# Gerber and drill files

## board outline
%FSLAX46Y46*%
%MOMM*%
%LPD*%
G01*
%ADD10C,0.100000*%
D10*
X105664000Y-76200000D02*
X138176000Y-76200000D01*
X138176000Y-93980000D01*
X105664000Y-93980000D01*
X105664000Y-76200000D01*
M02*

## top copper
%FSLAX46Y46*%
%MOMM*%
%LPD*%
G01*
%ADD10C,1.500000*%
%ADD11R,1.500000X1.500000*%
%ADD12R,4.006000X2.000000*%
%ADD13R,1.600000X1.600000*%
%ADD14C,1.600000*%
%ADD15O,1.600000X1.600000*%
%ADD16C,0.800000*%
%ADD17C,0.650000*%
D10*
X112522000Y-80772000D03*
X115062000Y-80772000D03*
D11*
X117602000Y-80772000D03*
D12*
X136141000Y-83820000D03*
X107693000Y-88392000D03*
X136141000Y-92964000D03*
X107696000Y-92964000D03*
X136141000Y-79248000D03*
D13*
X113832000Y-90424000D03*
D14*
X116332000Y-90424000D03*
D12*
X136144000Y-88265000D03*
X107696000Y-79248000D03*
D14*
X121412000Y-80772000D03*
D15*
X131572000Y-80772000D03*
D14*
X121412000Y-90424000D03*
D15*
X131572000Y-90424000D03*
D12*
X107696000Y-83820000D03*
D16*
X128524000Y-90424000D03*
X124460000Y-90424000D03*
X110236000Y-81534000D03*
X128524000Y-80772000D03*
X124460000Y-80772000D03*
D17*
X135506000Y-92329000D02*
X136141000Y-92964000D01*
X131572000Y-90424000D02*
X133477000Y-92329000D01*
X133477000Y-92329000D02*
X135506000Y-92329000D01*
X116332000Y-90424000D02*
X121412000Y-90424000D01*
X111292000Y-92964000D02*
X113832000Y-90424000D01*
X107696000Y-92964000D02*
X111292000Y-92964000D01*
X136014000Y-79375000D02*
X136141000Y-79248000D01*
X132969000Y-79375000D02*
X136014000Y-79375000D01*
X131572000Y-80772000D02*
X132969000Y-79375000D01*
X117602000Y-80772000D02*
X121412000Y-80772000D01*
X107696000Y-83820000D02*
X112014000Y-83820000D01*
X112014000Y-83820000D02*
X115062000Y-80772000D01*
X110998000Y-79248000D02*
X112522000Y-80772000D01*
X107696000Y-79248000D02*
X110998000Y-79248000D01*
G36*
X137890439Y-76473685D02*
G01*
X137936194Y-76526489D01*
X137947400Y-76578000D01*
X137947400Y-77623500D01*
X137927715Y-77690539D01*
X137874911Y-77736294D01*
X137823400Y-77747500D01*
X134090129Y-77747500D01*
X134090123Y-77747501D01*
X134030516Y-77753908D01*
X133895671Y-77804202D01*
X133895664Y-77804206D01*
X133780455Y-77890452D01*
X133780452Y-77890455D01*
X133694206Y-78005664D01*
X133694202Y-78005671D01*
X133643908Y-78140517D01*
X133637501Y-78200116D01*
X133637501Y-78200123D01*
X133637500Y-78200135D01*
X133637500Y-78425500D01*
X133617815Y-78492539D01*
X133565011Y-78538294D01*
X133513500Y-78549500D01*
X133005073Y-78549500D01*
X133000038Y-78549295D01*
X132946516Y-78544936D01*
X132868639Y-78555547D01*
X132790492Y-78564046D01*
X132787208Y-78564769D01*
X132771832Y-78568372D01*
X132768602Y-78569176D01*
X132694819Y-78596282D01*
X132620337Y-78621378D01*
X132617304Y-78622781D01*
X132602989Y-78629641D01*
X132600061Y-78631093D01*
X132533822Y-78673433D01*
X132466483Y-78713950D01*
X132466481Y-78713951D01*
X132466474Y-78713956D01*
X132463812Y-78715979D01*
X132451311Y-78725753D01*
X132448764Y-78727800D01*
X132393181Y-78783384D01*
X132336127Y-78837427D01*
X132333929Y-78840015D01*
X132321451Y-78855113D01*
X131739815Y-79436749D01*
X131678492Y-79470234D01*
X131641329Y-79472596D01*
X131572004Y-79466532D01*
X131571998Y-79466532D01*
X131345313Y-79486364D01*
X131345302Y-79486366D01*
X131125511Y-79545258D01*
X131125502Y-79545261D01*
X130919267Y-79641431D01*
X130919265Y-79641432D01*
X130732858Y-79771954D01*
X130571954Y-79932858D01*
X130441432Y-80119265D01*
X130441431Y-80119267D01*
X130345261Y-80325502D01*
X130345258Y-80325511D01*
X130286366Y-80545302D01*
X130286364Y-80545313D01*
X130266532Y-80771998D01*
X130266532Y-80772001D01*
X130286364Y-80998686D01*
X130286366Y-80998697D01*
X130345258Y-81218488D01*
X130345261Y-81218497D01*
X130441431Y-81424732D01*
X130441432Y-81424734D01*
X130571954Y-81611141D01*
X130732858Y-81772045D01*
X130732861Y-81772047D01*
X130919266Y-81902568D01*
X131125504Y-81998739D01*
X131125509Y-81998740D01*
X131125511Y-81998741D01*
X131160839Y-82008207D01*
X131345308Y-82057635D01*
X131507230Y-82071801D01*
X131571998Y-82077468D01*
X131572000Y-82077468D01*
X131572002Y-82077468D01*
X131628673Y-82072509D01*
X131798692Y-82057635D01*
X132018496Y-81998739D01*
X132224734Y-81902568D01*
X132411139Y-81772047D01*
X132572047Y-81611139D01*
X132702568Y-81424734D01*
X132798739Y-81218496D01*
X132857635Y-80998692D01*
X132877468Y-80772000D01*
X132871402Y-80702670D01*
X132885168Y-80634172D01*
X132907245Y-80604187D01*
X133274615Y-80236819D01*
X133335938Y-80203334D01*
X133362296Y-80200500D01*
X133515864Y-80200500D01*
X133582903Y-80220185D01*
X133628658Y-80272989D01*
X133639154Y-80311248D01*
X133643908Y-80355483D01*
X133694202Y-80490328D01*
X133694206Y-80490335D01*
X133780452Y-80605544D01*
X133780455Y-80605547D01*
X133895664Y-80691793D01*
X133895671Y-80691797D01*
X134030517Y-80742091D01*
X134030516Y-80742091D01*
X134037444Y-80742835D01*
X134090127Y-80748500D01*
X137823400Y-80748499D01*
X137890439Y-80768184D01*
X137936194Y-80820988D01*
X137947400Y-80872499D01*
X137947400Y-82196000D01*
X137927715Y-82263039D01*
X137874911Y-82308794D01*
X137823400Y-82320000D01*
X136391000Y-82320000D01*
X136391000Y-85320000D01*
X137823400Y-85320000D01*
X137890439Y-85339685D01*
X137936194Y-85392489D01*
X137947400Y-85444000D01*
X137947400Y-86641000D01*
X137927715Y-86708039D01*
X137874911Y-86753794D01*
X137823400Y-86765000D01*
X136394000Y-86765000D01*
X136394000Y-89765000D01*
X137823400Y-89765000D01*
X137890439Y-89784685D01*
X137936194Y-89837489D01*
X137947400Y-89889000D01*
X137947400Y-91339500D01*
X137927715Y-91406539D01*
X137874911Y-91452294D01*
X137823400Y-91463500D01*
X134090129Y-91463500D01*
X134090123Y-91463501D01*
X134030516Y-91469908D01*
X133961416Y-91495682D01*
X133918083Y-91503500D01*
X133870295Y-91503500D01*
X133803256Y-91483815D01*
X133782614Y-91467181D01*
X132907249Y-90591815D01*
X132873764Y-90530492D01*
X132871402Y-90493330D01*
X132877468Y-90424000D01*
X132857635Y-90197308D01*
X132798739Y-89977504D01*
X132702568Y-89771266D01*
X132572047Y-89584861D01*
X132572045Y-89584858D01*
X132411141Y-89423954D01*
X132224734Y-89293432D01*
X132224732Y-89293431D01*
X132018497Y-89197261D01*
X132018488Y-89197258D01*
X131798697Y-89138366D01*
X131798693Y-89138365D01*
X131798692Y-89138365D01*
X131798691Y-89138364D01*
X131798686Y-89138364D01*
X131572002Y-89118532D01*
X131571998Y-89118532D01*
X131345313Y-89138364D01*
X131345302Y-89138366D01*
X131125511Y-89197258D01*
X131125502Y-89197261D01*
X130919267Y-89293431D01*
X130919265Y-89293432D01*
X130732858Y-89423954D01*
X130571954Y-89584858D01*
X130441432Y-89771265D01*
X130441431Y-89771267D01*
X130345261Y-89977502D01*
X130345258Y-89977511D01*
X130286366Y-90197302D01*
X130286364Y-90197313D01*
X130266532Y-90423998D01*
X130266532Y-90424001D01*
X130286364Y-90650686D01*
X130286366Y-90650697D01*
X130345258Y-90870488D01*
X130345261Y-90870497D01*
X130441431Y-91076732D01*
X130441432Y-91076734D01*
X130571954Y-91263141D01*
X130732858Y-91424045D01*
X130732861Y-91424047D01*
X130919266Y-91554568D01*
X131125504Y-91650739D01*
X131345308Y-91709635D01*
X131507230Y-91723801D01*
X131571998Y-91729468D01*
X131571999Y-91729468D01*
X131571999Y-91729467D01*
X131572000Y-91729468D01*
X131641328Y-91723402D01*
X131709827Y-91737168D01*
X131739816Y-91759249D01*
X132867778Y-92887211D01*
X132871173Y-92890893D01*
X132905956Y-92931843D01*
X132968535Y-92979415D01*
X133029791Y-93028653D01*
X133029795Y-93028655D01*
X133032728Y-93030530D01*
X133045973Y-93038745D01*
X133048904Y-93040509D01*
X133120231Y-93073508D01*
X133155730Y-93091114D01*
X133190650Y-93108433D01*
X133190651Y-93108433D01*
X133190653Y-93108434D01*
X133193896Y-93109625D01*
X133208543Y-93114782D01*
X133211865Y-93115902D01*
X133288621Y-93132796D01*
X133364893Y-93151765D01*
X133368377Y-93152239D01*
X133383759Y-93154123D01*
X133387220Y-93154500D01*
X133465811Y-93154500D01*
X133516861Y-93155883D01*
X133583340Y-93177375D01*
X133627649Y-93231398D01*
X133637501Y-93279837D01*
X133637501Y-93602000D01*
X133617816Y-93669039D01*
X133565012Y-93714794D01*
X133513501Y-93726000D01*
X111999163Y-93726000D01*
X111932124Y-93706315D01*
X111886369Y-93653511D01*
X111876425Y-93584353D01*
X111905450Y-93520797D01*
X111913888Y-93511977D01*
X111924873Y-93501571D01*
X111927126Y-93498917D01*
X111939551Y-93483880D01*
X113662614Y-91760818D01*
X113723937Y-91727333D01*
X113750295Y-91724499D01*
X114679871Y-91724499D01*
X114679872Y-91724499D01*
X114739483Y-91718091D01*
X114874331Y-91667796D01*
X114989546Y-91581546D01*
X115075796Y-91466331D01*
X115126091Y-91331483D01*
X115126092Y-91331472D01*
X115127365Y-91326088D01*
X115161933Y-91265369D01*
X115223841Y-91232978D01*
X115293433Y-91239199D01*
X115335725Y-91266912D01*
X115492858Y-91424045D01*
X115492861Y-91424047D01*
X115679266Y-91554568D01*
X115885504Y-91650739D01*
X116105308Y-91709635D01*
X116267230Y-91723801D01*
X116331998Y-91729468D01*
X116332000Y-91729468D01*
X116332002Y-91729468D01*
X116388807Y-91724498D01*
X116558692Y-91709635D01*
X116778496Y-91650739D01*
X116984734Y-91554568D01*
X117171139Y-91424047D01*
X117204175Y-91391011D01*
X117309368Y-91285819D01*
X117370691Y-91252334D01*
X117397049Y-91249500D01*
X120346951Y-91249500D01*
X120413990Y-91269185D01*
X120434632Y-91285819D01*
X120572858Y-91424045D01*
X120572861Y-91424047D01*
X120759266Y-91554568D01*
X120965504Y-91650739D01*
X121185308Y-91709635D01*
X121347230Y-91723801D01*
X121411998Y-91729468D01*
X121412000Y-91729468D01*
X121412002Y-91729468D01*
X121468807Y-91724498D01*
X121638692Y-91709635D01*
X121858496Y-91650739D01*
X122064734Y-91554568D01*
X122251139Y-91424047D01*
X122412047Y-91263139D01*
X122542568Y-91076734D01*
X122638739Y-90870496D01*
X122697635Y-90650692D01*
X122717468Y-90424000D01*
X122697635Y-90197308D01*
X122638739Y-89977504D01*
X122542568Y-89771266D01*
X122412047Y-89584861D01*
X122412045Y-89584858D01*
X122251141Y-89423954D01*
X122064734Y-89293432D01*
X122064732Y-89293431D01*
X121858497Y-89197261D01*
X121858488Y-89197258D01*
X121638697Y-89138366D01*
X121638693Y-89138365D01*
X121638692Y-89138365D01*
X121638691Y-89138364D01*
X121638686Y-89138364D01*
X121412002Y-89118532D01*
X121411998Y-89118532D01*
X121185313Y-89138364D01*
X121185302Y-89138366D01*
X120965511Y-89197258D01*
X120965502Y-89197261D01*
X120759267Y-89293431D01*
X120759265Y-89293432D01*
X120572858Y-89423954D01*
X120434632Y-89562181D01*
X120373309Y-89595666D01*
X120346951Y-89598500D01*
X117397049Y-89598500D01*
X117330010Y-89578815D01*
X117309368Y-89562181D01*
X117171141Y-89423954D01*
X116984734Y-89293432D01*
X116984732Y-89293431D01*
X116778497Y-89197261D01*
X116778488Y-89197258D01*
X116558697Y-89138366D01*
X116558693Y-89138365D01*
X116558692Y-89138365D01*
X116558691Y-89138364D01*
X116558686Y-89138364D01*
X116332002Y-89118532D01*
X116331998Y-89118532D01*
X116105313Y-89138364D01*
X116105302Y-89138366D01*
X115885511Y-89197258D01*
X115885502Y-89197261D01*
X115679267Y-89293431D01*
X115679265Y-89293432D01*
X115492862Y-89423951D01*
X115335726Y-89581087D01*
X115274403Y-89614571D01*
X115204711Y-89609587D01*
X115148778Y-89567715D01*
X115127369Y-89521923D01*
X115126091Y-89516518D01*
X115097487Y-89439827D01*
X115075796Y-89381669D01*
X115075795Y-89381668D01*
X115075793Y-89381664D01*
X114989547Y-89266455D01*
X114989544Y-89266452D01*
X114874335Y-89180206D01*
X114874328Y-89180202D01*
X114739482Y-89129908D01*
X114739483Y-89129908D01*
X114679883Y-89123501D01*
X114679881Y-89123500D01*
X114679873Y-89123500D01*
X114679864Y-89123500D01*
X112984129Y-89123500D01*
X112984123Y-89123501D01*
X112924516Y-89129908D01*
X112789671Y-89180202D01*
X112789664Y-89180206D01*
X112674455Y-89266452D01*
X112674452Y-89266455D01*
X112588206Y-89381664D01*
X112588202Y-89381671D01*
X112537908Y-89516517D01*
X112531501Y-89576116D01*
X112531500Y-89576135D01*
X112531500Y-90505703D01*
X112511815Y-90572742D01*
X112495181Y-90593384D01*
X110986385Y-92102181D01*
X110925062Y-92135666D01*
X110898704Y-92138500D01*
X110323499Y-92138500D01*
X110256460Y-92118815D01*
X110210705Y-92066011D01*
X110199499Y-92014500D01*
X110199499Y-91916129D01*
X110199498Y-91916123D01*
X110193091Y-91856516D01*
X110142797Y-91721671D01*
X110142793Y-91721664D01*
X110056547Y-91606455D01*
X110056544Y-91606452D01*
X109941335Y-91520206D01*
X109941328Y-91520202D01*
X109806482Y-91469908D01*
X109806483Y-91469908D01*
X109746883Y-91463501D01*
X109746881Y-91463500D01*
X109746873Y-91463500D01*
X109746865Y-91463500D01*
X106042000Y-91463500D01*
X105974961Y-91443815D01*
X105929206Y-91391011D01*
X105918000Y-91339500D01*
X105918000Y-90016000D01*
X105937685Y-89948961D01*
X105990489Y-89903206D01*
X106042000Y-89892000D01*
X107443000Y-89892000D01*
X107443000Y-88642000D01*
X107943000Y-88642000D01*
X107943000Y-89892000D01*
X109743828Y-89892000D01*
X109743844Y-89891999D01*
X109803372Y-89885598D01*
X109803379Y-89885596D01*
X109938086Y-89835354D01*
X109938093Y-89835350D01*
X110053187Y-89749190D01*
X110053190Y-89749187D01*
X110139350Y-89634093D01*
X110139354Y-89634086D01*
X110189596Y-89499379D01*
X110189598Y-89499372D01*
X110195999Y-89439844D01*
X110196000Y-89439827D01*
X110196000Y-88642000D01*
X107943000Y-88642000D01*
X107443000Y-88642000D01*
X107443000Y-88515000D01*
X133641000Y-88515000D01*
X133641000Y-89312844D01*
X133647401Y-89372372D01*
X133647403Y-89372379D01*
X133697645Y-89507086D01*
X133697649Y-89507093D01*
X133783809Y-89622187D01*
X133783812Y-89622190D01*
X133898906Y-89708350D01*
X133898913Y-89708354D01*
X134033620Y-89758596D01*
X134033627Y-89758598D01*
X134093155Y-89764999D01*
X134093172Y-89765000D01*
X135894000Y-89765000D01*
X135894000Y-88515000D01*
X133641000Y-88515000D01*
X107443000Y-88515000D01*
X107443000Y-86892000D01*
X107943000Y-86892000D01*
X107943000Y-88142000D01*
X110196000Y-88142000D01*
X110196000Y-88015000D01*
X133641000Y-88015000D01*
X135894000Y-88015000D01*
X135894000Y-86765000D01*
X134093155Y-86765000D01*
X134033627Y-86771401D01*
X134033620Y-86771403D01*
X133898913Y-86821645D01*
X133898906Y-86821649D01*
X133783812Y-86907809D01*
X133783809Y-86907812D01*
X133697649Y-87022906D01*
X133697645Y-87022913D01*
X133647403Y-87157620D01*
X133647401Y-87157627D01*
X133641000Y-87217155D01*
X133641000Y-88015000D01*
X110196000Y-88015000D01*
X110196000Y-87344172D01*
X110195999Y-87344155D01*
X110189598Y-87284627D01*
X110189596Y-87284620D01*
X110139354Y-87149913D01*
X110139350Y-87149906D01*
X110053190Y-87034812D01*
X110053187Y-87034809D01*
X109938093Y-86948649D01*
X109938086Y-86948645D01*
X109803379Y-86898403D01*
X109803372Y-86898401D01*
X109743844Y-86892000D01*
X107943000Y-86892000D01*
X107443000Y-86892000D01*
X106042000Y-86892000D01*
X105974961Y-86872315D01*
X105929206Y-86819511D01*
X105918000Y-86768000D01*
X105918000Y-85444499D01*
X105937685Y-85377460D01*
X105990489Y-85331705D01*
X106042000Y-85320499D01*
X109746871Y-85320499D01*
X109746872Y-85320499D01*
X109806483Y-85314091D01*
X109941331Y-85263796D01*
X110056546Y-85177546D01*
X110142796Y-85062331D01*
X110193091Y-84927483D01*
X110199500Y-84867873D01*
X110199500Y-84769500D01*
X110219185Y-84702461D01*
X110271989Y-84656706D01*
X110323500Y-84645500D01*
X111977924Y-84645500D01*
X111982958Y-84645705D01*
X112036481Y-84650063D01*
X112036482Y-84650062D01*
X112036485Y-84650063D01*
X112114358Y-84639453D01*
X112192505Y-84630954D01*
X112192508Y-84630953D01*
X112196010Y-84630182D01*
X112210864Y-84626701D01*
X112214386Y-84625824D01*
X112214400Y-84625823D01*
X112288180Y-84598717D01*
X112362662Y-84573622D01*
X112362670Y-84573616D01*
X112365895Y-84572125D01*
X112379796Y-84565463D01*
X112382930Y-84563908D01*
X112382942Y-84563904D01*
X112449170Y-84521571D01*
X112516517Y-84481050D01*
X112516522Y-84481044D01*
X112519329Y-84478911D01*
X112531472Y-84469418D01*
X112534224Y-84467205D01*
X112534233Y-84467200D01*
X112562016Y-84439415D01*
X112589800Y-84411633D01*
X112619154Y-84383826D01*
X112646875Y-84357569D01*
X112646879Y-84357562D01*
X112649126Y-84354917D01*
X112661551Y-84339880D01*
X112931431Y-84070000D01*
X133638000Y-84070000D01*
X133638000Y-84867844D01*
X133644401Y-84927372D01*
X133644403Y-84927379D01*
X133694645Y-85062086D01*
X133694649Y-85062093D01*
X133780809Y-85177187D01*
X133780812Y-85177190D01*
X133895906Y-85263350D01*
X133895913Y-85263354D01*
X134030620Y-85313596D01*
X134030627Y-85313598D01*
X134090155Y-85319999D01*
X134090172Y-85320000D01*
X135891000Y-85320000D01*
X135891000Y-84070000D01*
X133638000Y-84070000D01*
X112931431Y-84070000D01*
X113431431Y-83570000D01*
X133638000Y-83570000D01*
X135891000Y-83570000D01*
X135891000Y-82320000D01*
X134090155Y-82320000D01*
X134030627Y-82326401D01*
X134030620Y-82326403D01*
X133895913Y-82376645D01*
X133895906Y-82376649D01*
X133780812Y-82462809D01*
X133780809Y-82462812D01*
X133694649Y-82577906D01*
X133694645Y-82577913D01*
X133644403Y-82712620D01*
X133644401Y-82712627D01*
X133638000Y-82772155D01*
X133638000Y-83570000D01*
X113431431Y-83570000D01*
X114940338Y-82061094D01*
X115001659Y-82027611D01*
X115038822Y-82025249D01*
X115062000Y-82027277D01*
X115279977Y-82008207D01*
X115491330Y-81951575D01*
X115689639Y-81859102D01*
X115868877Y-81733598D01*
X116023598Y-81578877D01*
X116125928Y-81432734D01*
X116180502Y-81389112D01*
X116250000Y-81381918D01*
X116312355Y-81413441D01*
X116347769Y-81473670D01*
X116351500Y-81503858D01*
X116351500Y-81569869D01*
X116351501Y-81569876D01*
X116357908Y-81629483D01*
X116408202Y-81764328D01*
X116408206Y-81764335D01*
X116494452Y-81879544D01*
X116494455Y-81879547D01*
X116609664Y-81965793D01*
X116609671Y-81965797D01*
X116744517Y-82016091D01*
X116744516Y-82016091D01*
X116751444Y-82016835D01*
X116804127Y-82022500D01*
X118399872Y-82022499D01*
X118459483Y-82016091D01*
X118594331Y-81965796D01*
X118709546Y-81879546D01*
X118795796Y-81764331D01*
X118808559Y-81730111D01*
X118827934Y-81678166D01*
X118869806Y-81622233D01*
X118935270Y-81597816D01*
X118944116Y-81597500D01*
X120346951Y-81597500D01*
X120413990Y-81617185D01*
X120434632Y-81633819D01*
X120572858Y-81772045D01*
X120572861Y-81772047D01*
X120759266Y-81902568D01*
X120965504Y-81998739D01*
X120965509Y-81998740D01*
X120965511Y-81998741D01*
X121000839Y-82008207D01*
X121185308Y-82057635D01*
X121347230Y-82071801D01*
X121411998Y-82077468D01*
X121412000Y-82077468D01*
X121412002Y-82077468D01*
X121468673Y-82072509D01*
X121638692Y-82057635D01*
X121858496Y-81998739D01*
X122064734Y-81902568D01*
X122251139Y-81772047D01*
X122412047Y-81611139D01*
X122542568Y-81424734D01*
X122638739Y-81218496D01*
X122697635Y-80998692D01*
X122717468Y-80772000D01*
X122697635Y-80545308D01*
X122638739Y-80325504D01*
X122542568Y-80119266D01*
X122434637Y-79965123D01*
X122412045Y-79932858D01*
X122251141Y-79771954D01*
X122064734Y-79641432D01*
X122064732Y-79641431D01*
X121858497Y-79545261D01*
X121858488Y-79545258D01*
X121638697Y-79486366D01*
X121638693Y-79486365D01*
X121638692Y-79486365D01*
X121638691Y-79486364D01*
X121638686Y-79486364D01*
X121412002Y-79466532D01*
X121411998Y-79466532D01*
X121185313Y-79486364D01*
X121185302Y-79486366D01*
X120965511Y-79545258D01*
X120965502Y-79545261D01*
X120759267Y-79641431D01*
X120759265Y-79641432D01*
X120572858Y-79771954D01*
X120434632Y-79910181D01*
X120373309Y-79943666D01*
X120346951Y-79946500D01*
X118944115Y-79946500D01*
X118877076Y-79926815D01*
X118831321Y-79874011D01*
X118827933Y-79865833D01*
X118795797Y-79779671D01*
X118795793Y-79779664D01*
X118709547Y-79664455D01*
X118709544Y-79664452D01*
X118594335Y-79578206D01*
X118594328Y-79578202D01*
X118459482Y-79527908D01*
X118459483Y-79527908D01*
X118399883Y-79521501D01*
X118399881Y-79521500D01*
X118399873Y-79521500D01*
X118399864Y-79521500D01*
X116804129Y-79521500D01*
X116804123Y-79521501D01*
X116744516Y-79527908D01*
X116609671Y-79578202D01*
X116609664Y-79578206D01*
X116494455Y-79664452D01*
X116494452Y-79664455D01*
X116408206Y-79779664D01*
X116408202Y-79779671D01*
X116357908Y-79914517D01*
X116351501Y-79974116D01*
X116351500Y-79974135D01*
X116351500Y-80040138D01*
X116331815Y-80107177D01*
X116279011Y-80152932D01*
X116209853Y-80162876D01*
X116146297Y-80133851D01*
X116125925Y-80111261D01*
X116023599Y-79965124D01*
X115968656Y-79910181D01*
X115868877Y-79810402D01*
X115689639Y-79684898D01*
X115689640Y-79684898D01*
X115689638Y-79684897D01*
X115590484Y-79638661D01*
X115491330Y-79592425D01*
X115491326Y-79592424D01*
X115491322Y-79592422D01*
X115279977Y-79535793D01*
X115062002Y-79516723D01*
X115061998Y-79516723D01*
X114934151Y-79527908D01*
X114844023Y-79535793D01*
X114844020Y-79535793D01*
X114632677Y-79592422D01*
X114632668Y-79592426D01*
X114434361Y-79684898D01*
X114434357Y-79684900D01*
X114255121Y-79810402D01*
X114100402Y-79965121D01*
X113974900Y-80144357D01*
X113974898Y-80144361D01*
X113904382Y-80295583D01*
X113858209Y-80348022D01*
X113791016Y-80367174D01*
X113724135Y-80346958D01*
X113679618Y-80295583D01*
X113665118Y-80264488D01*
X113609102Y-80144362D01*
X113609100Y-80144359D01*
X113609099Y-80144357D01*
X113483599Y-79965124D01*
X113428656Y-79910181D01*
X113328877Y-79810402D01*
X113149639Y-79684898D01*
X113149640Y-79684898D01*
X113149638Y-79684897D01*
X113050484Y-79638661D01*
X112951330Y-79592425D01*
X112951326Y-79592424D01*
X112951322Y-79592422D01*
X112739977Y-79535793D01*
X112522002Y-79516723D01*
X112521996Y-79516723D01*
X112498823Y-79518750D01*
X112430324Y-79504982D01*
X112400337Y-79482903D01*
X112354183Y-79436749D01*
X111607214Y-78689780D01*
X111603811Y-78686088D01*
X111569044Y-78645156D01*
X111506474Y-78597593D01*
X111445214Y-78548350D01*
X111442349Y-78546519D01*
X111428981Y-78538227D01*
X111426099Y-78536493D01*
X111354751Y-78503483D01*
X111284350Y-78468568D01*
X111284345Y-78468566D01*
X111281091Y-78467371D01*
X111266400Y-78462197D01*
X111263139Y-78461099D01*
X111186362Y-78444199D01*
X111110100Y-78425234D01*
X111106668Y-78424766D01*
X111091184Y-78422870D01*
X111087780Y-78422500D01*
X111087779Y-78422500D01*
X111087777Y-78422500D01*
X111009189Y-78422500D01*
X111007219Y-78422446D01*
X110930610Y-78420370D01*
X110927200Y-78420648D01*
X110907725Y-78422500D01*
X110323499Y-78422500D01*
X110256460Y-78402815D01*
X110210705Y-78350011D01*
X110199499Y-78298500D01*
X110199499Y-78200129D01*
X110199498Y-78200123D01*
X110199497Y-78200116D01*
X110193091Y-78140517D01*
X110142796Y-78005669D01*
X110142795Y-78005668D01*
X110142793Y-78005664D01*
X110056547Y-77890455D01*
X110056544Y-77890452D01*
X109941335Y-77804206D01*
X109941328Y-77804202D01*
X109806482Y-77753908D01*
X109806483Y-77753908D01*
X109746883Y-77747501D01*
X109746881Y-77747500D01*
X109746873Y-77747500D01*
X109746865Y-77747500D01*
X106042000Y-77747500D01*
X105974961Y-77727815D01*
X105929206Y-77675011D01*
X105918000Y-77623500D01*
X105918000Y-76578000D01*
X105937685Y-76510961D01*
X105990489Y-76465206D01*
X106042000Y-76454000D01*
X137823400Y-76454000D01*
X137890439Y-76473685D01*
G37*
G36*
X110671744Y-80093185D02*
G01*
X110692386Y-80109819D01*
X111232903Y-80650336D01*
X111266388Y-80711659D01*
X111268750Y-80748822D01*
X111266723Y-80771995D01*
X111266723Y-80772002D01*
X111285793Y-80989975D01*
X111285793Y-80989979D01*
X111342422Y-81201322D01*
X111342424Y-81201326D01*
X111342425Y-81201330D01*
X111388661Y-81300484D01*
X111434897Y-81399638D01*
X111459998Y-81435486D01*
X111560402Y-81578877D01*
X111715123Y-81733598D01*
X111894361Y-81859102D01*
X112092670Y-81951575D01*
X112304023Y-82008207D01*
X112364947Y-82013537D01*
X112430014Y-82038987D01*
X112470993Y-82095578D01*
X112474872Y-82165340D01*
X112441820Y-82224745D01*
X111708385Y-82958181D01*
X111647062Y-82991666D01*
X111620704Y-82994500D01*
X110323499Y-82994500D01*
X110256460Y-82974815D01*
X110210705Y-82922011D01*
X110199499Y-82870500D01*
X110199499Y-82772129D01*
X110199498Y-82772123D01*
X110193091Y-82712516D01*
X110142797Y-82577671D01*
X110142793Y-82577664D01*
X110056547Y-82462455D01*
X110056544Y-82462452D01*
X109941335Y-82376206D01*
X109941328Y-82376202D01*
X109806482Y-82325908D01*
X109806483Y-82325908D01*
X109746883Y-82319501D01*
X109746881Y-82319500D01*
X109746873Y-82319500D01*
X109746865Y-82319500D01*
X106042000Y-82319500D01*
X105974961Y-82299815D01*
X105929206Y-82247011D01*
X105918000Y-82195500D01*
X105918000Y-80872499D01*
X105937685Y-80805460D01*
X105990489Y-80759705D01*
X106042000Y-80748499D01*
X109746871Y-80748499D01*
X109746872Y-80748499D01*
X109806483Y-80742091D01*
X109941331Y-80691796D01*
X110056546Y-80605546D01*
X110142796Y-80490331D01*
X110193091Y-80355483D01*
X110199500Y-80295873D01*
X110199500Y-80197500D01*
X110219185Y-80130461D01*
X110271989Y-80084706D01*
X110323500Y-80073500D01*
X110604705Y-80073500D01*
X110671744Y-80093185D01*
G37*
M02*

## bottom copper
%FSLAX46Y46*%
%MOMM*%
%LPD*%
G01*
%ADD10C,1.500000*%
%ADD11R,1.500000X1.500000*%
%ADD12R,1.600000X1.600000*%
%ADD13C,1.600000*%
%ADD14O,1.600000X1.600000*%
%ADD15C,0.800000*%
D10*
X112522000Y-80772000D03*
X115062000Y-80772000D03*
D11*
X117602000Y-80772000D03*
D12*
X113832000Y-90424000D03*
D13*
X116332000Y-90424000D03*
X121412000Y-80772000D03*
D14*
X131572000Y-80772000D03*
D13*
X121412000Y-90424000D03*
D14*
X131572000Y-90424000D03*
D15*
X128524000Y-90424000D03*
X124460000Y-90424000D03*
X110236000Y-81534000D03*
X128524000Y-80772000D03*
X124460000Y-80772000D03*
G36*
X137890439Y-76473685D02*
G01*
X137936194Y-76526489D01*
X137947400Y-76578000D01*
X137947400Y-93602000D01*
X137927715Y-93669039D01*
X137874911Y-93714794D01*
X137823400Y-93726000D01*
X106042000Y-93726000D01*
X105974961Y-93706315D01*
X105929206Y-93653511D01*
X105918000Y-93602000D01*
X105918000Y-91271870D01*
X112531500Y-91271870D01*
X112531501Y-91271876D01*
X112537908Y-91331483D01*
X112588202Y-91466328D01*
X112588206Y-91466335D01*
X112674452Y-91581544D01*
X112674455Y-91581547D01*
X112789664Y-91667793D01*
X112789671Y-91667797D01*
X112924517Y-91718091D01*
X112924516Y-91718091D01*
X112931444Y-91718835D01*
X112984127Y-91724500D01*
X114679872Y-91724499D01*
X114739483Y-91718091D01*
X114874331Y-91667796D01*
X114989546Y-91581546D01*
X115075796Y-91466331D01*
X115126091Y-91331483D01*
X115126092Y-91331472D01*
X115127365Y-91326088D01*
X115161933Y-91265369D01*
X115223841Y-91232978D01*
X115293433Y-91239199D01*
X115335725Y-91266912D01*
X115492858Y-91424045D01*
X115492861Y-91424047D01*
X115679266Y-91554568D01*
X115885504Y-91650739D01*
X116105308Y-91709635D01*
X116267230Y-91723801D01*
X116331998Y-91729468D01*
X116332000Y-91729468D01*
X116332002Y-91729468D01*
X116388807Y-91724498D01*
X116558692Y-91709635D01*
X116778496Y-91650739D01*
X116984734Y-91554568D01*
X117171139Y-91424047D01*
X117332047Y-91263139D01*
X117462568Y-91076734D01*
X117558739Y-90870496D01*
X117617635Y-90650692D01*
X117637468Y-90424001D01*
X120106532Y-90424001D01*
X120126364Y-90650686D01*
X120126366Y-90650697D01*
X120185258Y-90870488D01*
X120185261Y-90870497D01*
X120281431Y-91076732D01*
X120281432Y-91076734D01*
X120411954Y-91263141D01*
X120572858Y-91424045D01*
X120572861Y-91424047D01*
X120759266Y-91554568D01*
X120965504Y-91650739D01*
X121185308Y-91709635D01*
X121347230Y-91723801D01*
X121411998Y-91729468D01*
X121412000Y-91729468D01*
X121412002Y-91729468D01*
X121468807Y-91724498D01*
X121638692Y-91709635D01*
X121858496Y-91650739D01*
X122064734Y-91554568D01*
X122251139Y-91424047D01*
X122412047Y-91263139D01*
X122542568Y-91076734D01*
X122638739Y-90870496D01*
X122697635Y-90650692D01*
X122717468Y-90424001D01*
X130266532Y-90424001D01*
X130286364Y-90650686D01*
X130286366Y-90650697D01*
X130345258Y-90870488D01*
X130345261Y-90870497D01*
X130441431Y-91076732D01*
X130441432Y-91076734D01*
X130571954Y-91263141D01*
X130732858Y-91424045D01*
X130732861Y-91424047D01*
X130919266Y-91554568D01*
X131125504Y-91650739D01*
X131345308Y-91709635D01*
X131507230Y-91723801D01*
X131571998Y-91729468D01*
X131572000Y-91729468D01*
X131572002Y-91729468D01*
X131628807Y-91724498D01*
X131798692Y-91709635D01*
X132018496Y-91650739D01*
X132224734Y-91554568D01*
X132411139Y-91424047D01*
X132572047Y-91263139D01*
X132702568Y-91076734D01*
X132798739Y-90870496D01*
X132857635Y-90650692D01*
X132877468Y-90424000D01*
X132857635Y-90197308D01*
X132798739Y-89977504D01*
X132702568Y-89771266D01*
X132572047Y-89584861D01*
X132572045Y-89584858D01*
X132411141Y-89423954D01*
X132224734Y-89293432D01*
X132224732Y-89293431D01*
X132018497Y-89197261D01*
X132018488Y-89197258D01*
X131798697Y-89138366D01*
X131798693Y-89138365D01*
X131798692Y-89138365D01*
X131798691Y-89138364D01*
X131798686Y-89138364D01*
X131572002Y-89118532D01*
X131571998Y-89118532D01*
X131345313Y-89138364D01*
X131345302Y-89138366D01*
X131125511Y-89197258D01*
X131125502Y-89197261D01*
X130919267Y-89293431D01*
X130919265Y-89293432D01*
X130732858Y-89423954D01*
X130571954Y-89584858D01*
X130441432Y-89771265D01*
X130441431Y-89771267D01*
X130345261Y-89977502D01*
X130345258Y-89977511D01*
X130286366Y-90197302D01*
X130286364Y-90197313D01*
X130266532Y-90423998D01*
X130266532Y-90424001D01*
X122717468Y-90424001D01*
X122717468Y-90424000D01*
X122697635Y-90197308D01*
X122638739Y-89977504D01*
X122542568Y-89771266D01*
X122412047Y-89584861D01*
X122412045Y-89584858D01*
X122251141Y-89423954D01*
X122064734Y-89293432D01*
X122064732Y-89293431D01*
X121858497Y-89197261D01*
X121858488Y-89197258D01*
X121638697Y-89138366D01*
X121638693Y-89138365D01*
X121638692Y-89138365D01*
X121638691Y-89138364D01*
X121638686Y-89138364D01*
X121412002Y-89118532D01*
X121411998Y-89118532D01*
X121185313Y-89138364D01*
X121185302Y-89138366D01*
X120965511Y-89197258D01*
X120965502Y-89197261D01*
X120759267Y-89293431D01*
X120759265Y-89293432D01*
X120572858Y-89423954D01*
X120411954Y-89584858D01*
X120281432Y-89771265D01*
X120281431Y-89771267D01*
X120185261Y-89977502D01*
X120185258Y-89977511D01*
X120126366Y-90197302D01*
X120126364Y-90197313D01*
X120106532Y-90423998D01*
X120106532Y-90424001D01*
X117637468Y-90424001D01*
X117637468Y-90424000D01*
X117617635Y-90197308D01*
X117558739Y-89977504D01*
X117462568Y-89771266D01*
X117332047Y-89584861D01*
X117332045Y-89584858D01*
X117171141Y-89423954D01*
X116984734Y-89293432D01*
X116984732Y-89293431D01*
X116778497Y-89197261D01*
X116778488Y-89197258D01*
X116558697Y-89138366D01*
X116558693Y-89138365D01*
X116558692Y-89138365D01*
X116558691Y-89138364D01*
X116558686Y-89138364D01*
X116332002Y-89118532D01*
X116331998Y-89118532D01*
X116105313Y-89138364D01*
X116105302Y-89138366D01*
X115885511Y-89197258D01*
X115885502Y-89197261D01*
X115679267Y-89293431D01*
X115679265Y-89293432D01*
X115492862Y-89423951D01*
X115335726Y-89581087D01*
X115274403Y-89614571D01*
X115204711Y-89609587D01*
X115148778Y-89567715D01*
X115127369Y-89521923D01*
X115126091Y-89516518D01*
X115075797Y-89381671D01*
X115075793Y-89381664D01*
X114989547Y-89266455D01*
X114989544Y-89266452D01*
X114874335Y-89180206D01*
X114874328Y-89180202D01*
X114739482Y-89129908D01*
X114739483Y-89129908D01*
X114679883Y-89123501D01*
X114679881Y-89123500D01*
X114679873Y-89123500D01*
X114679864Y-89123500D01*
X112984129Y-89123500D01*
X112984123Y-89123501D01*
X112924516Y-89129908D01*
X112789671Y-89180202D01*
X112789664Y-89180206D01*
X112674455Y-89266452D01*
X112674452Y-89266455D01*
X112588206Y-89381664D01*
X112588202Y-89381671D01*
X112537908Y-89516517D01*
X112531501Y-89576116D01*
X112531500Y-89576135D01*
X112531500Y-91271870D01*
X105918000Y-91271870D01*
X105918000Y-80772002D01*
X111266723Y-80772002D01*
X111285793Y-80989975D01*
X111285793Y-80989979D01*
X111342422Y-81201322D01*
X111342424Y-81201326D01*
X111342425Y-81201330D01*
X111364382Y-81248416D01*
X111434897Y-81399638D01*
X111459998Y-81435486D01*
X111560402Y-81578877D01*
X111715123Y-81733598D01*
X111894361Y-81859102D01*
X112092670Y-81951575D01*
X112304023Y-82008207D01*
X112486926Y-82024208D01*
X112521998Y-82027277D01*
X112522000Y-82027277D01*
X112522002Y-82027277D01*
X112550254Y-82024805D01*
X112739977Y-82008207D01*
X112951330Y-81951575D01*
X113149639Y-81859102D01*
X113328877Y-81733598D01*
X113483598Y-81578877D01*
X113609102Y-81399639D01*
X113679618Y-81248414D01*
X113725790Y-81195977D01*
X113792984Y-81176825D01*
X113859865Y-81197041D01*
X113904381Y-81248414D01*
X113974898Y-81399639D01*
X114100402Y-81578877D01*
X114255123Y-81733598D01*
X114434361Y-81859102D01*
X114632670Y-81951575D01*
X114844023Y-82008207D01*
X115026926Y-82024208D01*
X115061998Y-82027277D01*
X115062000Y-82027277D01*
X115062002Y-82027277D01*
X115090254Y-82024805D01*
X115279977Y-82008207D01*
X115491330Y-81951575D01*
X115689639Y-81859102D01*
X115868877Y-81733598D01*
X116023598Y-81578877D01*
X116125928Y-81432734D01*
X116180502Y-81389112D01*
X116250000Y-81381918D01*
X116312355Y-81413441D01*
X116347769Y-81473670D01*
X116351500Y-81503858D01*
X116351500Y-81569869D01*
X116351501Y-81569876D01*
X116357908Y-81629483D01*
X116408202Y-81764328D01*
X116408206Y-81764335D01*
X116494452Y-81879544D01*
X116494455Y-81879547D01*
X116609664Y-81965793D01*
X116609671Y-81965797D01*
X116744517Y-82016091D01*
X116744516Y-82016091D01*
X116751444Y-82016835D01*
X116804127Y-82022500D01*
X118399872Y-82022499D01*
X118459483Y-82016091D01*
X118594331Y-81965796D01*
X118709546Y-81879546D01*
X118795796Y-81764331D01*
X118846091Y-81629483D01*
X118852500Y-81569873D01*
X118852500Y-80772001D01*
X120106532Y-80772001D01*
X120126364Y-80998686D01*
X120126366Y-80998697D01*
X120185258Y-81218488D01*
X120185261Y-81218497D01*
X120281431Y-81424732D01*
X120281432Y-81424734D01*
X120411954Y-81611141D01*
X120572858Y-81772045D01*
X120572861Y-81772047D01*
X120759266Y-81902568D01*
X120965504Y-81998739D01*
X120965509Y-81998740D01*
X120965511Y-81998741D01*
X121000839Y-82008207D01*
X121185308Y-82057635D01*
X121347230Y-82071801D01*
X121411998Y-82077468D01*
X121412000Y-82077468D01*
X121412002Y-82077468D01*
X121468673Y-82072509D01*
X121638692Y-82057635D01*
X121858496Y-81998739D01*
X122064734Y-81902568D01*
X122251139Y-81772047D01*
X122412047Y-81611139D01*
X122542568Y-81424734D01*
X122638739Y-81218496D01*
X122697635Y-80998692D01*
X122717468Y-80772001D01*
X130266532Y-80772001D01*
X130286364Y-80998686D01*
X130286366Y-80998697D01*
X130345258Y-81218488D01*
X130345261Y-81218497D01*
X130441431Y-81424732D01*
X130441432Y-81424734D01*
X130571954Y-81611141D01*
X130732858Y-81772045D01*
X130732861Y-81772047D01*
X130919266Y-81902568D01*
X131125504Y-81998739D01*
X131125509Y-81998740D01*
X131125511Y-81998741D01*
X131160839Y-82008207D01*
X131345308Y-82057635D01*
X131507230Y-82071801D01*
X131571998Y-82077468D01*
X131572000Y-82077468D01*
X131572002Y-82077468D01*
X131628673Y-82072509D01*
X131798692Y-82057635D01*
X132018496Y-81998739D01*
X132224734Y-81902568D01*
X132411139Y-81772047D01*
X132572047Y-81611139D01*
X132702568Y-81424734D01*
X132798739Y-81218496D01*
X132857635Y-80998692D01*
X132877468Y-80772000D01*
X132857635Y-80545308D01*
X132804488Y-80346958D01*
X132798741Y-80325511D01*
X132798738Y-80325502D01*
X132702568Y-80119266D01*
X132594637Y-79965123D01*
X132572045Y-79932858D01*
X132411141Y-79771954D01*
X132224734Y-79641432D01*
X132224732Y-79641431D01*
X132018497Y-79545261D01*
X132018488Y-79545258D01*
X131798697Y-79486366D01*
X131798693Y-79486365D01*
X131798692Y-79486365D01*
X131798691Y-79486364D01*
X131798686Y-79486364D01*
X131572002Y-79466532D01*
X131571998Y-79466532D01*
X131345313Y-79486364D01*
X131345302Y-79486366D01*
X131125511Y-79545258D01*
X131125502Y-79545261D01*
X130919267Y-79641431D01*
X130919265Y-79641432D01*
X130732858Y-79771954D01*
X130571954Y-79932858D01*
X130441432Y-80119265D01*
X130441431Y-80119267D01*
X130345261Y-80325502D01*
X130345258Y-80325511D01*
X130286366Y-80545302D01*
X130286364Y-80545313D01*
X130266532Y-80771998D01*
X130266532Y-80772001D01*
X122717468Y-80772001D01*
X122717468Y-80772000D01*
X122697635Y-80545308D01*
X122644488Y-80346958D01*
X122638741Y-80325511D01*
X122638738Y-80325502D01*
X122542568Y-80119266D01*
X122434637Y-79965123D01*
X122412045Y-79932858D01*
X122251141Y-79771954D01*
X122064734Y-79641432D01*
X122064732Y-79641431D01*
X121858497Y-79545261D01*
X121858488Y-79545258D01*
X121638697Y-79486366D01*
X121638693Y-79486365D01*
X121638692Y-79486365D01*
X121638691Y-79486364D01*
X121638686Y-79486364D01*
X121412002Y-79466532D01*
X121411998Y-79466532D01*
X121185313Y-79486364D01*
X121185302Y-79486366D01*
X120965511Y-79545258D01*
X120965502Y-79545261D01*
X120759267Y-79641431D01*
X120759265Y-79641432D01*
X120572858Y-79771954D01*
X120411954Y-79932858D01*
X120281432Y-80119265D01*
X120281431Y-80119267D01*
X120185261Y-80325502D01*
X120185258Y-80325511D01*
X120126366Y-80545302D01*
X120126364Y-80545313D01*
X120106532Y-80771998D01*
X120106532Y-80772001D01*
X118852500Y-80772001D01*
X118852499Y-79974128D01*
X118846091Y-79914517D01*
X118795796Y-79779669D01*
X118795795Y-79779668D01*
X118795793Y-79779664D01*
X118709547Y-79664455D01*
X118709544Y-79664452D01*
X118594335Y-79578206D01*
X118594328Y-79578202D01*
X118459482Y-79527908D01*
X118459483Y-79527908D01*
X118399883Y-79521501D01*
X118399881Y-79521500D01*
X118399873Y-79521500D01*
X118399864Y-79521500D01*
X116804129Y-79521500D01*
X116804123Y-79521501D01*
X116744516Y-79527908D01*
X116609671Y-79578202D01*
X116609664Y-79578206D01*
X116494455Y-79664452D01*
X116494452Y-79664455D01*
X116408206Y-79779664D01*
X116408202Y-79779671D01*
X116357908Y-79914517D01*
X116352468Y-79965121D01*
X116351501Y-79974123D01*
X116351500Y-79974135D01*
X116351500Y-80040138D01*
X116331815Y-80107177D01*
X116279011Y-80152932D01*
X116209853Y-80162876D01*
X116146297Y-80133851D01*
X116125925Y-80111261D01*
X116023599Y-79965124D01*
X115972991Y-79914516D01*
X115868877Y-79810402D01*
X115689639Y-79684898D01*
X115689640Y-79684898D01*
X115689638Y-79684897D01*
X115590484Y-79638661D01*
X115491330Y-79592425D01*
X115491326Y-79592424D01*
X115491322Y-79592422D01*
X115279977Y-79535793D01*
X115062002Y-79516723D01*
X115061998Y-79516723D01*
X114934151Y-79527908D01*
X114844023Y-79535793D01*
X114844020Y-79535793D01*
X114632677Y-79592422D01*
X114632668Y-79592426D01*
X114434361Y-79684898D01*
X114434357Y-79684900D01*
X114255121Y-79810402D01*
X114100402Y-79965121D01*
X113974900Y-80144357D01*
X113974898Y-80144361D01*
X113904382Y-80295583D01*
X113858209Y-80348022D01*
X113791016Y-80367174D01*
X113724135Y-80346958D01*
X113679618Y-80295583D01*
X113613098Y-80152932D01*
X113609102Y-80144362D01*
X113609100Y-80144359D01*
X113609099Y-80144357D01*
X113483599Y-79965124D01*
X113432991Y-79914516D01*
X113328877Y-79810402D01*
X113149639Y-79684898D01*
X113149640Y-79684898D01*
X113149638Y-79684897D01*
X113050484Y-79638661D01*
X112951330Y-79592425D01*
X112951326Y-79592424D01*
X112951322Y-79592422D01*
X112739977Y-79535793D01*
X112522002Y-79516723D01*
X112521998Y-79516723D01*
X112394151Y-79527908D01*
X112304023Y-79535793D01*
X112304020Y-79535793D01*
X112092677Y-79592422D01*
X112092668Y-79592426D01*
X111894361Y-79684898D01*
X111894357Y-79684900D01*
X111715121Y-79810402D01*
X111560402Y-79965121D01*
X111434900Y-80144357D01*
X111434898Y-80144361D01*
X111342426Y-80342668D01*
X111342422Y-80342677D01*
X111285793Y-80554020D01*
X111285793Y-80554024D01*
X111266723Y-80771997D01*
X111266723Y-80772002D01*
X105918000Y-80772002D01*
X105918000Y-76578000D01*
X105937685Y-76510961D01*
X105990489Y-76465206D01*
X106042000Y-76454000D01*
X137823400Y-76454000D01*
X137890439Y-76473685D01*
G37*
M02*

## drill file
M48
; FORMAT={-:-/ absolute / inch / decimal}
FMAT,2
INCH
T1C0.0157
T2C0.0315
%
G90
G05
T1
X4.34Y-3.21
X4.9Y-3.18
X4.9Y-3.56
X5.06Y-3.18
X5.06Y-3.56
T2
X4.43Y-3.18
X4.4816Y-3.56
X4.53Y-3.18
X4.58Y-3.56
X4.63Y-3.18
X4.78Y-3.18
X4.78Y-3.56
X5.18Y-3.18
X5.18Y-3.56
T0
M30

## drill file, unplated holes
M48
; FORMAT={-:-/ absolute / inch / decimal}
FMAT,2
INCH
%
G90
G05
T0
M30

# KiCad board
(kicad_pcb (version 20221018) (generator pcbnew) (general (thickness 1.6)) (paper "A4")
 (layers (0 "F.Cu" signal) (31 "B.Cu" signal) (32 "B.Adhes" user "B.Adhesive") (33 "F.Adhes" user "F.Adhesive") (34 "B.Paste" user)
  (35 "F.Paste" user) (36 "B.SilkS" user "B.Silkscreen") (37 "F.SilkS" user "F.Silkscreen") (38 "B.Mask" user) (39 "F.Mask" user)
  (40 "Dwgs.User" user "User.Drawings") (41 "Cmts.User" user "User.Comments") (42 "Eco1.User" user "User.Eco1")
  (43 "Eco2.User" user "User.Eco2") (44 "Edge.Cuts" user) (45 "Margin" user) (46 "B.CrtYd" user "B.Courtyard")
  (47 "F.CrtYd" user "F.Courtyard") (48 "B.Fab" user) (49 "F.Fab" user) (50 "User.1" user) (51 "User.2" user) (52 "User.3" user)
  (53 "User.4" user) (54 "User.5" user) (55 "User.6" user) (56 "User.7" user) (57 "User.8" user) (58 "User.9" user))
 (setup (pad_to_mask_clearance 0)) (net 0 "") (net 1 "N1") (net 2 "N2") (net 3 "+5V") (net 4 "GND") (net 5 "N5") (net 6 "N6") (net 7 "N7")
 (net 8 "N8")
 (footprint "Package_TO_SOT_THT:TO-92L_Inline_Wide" (layer "F.Cu") (at 117.602 80.772 180)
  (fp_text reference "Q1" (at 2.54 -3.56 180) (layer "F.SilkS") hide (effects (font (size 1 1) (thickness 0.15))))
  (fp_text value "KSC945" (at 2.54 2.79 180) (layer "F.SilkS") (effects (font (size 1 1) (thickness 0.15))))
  (pad "1" thru_hole rect (at 0 0 180) (size 1.5 1.5) (drill 0.8) (layers "*.Cu" "*.Mask") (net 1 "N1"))
  (pad "2" thru_hole circle (at 2.54 0 180) (size 1.5 1.5) (drill 0.8) (layers "*.Cu" "*.Mask") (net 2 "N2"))
  (pad "3" thru_hole circle (at 5.08 0 180) (size 1.5 1.5) (drill 0.8) (layers "*.Cu" "*.Mask") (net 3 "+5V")))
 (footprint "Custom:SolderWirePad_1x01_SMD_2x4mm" (layer "F.Cu") (at 136.144 83.82 90)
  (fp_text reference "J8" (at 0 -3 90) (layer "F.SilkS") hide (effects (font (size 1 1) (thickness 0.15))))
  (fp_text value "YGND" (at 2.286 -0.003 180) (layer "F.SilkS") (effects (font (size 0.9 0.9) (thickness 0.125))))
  (pad "1" smd rect (at 0 -0.003 90) (size 2 4.006) (layers "F.Cu" "F.Paste" "F.Mask") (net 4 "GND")))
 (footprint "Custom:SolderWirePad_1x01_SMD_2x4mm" (layer "F.Cu") (at 107.69 88.392 -90)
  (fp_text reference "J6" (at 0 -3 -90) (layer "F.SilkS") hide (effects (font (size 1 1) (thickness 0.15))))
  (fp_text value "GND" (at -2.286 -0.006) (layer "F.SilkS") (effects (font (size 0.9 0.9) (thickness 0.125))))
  (pad "1" smd rect (at 0 -0.003 270) (size 2 4.006) (layers "F.Cu" "F.Paste" "F.Mask") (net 4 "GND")))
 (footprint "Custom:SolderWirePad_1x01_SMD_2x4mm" (layer "F.Cu") (at 136.144 92.964 90)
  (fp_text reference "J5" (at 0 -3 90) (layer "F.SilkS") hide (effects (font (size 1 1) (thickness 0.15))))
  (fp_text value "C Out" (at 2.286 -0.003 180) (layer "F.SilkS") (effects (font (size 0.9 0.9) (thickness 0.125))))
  (pad "1" smd rect (at 0 -0.003 90) (size 2 4.006) (layers "F.Cu" "F.Paste" "F.Mask") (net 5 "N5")))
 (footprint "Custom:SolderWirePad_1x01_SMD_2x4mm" (layer "F.Cu") (at 107.693 92.964 -90)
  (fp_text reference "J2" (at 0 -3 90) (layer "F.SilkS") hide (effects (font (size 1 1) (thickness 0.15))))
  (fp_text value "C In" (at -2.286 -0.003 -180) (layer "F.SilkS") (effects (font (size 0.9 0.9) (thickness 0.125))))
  (pad "1" smd rect (at 0 -0.003 270) (size 2 4.006) (layers "F.Cu" "F.Paste" "F.Mask") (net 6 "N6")))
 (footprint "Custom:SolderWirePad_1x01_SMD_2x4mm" (layer "F.Cu") (at 136.144 79.248 90)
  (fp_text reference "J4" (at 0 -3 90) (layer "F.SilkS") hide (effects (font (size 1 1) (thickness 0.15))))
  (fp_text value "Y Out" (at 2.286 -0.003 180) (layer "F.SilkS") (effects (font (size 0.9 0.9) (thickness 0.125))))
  (pad "1" smd rect (at 0 -0.003 90) (size 2 4.006) (layers "F.Cu" "F.Paste" "F.Mask") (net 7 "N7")))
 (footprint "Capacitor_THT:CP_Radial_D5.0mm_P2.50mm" (layer "F.Cu") (at 113.832 90.424)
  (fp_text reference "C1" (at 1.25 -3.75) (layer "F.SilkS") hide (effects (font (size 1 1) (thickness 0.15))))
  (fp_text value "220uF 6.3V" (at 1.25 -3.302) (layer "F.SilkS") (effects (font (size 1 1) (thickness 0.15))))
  (pad "1" thru_hole rect (at 0 0) (size 1.6 1.6) (drill 0.8) (layers "*.Cu" "*.Mask") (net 6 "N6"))
  (pad "2" thru_hole circle (at 2.5 0) (size 1.6 1.6) (drill 0.8) (layers "*.Cu" "*.Mask") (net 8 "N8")))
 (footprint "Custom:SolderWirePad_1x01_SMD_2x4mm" (layer "F.Cu") (at 136.147 88.265 90)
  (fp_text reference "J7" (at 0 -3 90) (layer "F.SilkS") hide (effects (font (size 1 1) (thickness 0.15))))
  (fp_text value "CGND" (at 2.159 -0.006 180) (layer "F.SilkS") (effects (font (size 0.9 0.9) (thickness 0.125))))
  (pad "1" smd rect (at 0 -0.003 90) (size 2 4.006) (layers "F.Cu" "F.Paste" "F.Mask") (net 4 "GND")))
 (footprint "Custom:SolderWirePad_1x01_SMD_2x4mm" (layer "F.Cu") (at 107.693 79.248 -90)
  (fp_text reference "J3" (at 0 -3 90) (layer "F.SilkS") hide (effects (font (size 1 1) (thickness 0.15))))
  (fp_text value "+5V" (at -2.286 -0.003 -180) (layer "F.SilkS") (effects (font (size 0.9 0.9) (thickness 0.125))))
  (pad "1" smd rect (at 0 -0.003 270) (size 2 4.006) (layers "F.Cu" "F.Paste" "F.Mask") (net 3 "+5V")))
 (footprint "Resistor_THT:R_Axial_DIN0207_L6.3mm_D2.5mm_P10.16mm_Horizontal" (layer "F.Cu") (at 121.412 80.772)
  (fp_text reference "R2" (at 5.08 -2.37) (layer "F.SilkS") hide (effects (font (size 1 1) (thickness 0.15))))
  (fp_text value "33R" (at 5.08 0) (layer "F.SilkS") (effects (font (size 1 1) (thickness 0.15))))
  (pad "1" thru_hole circle (at 0 0) (size 1.6 1.6) (drill 0.8) (layers "*.Cu" "*.Mask") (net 1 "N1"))
  (pad "2" thru_hole oval (at 10.16 0) (size 1.6 1.6) (drill 0.8) (layers "*.Cu" "*.Mask") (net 7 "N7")))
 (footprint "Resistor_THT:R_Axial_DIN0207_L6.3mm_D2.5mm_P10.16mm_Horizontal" (layer "F.Cu") (at 121.412 90.424)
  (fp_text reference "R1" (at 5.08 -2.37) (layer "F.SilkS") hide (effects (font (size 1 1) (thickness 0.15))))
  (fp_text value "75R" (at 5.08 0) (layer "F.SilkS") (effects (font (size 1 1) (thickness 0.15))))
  (pad "1" thru_hole circle (at 0 0) (size 1.6 1.6) (drill 0.8) (layers "*.Cu" "*.Mask") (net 8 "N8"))
  (pad "2" thru_hole oval (at 10.16 0) (size 1.6 1.6) (drill 0.8) (layers "*.Cu" "*.Mask") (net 5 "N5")))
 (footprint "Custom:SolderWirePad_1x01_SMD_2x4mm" (layer "F.Cu") (at 107.693 83.82 -90)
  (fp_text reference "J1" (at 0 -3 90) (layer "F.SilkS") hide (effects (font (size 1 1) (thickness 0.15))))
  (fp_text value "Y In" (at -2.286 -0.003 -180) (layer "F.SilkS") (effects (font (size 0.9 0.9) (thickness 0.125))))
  (pad "1" smd rect (at 0 -0.003 270) (size 2 4.006) (layers "F.Cu" "F.Paste" "F.Mask") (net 2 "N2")))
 (gr_rect (start 105.664 76.2) (end 138.176 93.98) (stroke (width 0.1) (type default)) (fill none) (layer "Edge.Cuts"))
 (segment (start 111.292 92.964) (end 113.832 90.424) (width 0.65) (layer "F.Cu") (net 6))
 (segment (start 107.696 92.964) (end 111.292 92.964) (width 0.65) (layer "F.Cu") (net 6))
 (segment (start 116.332 90.424) (end 121.412 90.424) (width 0.65) (layer "F.Cu") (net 8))
 (segment (start 107.696 83.82) (end 112.014 83.82) (width 0.65) (layer "F.Cu") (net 2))
 (segment (start 112.014 83.82) (end 115.062 80.772) (width 0.65) (layer "F.Cu") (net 2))
 (segment (start 136.014 79.375) (end 136.141 79.248) (width 0.65) (layer "F.Cu") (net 7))
 (segment (start 131.572 80.772) (end 132.969 79.375) (width 0.65) (layer "F.Cu") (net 7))
 (segment (start 132.969 79.375) (end 136.014 79.375) (width 0.65) (layer "F.Cu") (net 7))
 (segment (start 133.477 92.329) (end 135.506 92.329) (width 0.65) (layer "F.Cu") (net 5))
 (segment (start 131.572 90.424) (end 133.477 92.329) (width 0.65) (layer "F.Cu") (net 5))
 (segment (start 135.506 92.329) (end 136.141 92.964) (width 0.65) (layer "F.Cu") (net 5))
 (segment (start 110.998 79.248) (end 112.522 80.772) (width 0.65) (layer "F.Cu") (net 3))
 (segment (start 107.696 79.248) (end 110.998 79.248) (width 0.65) (layer "F.Cu") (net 3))
 (segment (start 117.602 80.772) (end 121.412 80.772) (width 0.65) (layer "F.Cu") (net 1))
 (via (at 110.236 81.534) (size 0.8) (drill 0.4) (layers "F.Cu" "B.Cu") (free) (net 4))
 (via (at 124.46 80.772) (size 0.8) (drill 0.4) (layers "F.Cu" "B.Cu") (free) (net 4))
 (via (at 128.524 80.772) (size 0.8) (drill 0.4) (layers "F.Cu" "B.Cu") (free) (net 4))
 (via (at 128.524 90.424) (size 0.8) (drill 0.4) (layers "F.Cu" "B.Cu") (free) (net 4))
 (via (at 124.46 90.424) (size 0.8) (drill 0.4) (layers "F.Cu" "B.Cu") (free) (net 4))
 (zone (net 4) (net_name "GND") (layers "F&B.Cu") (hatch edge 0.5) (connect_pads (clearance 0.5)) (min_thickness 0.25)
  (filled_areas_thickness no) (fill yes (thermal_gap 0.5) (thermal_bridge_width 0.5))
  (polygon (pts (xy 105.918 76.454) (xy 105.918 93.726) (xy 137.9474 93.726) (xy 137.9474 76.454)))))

